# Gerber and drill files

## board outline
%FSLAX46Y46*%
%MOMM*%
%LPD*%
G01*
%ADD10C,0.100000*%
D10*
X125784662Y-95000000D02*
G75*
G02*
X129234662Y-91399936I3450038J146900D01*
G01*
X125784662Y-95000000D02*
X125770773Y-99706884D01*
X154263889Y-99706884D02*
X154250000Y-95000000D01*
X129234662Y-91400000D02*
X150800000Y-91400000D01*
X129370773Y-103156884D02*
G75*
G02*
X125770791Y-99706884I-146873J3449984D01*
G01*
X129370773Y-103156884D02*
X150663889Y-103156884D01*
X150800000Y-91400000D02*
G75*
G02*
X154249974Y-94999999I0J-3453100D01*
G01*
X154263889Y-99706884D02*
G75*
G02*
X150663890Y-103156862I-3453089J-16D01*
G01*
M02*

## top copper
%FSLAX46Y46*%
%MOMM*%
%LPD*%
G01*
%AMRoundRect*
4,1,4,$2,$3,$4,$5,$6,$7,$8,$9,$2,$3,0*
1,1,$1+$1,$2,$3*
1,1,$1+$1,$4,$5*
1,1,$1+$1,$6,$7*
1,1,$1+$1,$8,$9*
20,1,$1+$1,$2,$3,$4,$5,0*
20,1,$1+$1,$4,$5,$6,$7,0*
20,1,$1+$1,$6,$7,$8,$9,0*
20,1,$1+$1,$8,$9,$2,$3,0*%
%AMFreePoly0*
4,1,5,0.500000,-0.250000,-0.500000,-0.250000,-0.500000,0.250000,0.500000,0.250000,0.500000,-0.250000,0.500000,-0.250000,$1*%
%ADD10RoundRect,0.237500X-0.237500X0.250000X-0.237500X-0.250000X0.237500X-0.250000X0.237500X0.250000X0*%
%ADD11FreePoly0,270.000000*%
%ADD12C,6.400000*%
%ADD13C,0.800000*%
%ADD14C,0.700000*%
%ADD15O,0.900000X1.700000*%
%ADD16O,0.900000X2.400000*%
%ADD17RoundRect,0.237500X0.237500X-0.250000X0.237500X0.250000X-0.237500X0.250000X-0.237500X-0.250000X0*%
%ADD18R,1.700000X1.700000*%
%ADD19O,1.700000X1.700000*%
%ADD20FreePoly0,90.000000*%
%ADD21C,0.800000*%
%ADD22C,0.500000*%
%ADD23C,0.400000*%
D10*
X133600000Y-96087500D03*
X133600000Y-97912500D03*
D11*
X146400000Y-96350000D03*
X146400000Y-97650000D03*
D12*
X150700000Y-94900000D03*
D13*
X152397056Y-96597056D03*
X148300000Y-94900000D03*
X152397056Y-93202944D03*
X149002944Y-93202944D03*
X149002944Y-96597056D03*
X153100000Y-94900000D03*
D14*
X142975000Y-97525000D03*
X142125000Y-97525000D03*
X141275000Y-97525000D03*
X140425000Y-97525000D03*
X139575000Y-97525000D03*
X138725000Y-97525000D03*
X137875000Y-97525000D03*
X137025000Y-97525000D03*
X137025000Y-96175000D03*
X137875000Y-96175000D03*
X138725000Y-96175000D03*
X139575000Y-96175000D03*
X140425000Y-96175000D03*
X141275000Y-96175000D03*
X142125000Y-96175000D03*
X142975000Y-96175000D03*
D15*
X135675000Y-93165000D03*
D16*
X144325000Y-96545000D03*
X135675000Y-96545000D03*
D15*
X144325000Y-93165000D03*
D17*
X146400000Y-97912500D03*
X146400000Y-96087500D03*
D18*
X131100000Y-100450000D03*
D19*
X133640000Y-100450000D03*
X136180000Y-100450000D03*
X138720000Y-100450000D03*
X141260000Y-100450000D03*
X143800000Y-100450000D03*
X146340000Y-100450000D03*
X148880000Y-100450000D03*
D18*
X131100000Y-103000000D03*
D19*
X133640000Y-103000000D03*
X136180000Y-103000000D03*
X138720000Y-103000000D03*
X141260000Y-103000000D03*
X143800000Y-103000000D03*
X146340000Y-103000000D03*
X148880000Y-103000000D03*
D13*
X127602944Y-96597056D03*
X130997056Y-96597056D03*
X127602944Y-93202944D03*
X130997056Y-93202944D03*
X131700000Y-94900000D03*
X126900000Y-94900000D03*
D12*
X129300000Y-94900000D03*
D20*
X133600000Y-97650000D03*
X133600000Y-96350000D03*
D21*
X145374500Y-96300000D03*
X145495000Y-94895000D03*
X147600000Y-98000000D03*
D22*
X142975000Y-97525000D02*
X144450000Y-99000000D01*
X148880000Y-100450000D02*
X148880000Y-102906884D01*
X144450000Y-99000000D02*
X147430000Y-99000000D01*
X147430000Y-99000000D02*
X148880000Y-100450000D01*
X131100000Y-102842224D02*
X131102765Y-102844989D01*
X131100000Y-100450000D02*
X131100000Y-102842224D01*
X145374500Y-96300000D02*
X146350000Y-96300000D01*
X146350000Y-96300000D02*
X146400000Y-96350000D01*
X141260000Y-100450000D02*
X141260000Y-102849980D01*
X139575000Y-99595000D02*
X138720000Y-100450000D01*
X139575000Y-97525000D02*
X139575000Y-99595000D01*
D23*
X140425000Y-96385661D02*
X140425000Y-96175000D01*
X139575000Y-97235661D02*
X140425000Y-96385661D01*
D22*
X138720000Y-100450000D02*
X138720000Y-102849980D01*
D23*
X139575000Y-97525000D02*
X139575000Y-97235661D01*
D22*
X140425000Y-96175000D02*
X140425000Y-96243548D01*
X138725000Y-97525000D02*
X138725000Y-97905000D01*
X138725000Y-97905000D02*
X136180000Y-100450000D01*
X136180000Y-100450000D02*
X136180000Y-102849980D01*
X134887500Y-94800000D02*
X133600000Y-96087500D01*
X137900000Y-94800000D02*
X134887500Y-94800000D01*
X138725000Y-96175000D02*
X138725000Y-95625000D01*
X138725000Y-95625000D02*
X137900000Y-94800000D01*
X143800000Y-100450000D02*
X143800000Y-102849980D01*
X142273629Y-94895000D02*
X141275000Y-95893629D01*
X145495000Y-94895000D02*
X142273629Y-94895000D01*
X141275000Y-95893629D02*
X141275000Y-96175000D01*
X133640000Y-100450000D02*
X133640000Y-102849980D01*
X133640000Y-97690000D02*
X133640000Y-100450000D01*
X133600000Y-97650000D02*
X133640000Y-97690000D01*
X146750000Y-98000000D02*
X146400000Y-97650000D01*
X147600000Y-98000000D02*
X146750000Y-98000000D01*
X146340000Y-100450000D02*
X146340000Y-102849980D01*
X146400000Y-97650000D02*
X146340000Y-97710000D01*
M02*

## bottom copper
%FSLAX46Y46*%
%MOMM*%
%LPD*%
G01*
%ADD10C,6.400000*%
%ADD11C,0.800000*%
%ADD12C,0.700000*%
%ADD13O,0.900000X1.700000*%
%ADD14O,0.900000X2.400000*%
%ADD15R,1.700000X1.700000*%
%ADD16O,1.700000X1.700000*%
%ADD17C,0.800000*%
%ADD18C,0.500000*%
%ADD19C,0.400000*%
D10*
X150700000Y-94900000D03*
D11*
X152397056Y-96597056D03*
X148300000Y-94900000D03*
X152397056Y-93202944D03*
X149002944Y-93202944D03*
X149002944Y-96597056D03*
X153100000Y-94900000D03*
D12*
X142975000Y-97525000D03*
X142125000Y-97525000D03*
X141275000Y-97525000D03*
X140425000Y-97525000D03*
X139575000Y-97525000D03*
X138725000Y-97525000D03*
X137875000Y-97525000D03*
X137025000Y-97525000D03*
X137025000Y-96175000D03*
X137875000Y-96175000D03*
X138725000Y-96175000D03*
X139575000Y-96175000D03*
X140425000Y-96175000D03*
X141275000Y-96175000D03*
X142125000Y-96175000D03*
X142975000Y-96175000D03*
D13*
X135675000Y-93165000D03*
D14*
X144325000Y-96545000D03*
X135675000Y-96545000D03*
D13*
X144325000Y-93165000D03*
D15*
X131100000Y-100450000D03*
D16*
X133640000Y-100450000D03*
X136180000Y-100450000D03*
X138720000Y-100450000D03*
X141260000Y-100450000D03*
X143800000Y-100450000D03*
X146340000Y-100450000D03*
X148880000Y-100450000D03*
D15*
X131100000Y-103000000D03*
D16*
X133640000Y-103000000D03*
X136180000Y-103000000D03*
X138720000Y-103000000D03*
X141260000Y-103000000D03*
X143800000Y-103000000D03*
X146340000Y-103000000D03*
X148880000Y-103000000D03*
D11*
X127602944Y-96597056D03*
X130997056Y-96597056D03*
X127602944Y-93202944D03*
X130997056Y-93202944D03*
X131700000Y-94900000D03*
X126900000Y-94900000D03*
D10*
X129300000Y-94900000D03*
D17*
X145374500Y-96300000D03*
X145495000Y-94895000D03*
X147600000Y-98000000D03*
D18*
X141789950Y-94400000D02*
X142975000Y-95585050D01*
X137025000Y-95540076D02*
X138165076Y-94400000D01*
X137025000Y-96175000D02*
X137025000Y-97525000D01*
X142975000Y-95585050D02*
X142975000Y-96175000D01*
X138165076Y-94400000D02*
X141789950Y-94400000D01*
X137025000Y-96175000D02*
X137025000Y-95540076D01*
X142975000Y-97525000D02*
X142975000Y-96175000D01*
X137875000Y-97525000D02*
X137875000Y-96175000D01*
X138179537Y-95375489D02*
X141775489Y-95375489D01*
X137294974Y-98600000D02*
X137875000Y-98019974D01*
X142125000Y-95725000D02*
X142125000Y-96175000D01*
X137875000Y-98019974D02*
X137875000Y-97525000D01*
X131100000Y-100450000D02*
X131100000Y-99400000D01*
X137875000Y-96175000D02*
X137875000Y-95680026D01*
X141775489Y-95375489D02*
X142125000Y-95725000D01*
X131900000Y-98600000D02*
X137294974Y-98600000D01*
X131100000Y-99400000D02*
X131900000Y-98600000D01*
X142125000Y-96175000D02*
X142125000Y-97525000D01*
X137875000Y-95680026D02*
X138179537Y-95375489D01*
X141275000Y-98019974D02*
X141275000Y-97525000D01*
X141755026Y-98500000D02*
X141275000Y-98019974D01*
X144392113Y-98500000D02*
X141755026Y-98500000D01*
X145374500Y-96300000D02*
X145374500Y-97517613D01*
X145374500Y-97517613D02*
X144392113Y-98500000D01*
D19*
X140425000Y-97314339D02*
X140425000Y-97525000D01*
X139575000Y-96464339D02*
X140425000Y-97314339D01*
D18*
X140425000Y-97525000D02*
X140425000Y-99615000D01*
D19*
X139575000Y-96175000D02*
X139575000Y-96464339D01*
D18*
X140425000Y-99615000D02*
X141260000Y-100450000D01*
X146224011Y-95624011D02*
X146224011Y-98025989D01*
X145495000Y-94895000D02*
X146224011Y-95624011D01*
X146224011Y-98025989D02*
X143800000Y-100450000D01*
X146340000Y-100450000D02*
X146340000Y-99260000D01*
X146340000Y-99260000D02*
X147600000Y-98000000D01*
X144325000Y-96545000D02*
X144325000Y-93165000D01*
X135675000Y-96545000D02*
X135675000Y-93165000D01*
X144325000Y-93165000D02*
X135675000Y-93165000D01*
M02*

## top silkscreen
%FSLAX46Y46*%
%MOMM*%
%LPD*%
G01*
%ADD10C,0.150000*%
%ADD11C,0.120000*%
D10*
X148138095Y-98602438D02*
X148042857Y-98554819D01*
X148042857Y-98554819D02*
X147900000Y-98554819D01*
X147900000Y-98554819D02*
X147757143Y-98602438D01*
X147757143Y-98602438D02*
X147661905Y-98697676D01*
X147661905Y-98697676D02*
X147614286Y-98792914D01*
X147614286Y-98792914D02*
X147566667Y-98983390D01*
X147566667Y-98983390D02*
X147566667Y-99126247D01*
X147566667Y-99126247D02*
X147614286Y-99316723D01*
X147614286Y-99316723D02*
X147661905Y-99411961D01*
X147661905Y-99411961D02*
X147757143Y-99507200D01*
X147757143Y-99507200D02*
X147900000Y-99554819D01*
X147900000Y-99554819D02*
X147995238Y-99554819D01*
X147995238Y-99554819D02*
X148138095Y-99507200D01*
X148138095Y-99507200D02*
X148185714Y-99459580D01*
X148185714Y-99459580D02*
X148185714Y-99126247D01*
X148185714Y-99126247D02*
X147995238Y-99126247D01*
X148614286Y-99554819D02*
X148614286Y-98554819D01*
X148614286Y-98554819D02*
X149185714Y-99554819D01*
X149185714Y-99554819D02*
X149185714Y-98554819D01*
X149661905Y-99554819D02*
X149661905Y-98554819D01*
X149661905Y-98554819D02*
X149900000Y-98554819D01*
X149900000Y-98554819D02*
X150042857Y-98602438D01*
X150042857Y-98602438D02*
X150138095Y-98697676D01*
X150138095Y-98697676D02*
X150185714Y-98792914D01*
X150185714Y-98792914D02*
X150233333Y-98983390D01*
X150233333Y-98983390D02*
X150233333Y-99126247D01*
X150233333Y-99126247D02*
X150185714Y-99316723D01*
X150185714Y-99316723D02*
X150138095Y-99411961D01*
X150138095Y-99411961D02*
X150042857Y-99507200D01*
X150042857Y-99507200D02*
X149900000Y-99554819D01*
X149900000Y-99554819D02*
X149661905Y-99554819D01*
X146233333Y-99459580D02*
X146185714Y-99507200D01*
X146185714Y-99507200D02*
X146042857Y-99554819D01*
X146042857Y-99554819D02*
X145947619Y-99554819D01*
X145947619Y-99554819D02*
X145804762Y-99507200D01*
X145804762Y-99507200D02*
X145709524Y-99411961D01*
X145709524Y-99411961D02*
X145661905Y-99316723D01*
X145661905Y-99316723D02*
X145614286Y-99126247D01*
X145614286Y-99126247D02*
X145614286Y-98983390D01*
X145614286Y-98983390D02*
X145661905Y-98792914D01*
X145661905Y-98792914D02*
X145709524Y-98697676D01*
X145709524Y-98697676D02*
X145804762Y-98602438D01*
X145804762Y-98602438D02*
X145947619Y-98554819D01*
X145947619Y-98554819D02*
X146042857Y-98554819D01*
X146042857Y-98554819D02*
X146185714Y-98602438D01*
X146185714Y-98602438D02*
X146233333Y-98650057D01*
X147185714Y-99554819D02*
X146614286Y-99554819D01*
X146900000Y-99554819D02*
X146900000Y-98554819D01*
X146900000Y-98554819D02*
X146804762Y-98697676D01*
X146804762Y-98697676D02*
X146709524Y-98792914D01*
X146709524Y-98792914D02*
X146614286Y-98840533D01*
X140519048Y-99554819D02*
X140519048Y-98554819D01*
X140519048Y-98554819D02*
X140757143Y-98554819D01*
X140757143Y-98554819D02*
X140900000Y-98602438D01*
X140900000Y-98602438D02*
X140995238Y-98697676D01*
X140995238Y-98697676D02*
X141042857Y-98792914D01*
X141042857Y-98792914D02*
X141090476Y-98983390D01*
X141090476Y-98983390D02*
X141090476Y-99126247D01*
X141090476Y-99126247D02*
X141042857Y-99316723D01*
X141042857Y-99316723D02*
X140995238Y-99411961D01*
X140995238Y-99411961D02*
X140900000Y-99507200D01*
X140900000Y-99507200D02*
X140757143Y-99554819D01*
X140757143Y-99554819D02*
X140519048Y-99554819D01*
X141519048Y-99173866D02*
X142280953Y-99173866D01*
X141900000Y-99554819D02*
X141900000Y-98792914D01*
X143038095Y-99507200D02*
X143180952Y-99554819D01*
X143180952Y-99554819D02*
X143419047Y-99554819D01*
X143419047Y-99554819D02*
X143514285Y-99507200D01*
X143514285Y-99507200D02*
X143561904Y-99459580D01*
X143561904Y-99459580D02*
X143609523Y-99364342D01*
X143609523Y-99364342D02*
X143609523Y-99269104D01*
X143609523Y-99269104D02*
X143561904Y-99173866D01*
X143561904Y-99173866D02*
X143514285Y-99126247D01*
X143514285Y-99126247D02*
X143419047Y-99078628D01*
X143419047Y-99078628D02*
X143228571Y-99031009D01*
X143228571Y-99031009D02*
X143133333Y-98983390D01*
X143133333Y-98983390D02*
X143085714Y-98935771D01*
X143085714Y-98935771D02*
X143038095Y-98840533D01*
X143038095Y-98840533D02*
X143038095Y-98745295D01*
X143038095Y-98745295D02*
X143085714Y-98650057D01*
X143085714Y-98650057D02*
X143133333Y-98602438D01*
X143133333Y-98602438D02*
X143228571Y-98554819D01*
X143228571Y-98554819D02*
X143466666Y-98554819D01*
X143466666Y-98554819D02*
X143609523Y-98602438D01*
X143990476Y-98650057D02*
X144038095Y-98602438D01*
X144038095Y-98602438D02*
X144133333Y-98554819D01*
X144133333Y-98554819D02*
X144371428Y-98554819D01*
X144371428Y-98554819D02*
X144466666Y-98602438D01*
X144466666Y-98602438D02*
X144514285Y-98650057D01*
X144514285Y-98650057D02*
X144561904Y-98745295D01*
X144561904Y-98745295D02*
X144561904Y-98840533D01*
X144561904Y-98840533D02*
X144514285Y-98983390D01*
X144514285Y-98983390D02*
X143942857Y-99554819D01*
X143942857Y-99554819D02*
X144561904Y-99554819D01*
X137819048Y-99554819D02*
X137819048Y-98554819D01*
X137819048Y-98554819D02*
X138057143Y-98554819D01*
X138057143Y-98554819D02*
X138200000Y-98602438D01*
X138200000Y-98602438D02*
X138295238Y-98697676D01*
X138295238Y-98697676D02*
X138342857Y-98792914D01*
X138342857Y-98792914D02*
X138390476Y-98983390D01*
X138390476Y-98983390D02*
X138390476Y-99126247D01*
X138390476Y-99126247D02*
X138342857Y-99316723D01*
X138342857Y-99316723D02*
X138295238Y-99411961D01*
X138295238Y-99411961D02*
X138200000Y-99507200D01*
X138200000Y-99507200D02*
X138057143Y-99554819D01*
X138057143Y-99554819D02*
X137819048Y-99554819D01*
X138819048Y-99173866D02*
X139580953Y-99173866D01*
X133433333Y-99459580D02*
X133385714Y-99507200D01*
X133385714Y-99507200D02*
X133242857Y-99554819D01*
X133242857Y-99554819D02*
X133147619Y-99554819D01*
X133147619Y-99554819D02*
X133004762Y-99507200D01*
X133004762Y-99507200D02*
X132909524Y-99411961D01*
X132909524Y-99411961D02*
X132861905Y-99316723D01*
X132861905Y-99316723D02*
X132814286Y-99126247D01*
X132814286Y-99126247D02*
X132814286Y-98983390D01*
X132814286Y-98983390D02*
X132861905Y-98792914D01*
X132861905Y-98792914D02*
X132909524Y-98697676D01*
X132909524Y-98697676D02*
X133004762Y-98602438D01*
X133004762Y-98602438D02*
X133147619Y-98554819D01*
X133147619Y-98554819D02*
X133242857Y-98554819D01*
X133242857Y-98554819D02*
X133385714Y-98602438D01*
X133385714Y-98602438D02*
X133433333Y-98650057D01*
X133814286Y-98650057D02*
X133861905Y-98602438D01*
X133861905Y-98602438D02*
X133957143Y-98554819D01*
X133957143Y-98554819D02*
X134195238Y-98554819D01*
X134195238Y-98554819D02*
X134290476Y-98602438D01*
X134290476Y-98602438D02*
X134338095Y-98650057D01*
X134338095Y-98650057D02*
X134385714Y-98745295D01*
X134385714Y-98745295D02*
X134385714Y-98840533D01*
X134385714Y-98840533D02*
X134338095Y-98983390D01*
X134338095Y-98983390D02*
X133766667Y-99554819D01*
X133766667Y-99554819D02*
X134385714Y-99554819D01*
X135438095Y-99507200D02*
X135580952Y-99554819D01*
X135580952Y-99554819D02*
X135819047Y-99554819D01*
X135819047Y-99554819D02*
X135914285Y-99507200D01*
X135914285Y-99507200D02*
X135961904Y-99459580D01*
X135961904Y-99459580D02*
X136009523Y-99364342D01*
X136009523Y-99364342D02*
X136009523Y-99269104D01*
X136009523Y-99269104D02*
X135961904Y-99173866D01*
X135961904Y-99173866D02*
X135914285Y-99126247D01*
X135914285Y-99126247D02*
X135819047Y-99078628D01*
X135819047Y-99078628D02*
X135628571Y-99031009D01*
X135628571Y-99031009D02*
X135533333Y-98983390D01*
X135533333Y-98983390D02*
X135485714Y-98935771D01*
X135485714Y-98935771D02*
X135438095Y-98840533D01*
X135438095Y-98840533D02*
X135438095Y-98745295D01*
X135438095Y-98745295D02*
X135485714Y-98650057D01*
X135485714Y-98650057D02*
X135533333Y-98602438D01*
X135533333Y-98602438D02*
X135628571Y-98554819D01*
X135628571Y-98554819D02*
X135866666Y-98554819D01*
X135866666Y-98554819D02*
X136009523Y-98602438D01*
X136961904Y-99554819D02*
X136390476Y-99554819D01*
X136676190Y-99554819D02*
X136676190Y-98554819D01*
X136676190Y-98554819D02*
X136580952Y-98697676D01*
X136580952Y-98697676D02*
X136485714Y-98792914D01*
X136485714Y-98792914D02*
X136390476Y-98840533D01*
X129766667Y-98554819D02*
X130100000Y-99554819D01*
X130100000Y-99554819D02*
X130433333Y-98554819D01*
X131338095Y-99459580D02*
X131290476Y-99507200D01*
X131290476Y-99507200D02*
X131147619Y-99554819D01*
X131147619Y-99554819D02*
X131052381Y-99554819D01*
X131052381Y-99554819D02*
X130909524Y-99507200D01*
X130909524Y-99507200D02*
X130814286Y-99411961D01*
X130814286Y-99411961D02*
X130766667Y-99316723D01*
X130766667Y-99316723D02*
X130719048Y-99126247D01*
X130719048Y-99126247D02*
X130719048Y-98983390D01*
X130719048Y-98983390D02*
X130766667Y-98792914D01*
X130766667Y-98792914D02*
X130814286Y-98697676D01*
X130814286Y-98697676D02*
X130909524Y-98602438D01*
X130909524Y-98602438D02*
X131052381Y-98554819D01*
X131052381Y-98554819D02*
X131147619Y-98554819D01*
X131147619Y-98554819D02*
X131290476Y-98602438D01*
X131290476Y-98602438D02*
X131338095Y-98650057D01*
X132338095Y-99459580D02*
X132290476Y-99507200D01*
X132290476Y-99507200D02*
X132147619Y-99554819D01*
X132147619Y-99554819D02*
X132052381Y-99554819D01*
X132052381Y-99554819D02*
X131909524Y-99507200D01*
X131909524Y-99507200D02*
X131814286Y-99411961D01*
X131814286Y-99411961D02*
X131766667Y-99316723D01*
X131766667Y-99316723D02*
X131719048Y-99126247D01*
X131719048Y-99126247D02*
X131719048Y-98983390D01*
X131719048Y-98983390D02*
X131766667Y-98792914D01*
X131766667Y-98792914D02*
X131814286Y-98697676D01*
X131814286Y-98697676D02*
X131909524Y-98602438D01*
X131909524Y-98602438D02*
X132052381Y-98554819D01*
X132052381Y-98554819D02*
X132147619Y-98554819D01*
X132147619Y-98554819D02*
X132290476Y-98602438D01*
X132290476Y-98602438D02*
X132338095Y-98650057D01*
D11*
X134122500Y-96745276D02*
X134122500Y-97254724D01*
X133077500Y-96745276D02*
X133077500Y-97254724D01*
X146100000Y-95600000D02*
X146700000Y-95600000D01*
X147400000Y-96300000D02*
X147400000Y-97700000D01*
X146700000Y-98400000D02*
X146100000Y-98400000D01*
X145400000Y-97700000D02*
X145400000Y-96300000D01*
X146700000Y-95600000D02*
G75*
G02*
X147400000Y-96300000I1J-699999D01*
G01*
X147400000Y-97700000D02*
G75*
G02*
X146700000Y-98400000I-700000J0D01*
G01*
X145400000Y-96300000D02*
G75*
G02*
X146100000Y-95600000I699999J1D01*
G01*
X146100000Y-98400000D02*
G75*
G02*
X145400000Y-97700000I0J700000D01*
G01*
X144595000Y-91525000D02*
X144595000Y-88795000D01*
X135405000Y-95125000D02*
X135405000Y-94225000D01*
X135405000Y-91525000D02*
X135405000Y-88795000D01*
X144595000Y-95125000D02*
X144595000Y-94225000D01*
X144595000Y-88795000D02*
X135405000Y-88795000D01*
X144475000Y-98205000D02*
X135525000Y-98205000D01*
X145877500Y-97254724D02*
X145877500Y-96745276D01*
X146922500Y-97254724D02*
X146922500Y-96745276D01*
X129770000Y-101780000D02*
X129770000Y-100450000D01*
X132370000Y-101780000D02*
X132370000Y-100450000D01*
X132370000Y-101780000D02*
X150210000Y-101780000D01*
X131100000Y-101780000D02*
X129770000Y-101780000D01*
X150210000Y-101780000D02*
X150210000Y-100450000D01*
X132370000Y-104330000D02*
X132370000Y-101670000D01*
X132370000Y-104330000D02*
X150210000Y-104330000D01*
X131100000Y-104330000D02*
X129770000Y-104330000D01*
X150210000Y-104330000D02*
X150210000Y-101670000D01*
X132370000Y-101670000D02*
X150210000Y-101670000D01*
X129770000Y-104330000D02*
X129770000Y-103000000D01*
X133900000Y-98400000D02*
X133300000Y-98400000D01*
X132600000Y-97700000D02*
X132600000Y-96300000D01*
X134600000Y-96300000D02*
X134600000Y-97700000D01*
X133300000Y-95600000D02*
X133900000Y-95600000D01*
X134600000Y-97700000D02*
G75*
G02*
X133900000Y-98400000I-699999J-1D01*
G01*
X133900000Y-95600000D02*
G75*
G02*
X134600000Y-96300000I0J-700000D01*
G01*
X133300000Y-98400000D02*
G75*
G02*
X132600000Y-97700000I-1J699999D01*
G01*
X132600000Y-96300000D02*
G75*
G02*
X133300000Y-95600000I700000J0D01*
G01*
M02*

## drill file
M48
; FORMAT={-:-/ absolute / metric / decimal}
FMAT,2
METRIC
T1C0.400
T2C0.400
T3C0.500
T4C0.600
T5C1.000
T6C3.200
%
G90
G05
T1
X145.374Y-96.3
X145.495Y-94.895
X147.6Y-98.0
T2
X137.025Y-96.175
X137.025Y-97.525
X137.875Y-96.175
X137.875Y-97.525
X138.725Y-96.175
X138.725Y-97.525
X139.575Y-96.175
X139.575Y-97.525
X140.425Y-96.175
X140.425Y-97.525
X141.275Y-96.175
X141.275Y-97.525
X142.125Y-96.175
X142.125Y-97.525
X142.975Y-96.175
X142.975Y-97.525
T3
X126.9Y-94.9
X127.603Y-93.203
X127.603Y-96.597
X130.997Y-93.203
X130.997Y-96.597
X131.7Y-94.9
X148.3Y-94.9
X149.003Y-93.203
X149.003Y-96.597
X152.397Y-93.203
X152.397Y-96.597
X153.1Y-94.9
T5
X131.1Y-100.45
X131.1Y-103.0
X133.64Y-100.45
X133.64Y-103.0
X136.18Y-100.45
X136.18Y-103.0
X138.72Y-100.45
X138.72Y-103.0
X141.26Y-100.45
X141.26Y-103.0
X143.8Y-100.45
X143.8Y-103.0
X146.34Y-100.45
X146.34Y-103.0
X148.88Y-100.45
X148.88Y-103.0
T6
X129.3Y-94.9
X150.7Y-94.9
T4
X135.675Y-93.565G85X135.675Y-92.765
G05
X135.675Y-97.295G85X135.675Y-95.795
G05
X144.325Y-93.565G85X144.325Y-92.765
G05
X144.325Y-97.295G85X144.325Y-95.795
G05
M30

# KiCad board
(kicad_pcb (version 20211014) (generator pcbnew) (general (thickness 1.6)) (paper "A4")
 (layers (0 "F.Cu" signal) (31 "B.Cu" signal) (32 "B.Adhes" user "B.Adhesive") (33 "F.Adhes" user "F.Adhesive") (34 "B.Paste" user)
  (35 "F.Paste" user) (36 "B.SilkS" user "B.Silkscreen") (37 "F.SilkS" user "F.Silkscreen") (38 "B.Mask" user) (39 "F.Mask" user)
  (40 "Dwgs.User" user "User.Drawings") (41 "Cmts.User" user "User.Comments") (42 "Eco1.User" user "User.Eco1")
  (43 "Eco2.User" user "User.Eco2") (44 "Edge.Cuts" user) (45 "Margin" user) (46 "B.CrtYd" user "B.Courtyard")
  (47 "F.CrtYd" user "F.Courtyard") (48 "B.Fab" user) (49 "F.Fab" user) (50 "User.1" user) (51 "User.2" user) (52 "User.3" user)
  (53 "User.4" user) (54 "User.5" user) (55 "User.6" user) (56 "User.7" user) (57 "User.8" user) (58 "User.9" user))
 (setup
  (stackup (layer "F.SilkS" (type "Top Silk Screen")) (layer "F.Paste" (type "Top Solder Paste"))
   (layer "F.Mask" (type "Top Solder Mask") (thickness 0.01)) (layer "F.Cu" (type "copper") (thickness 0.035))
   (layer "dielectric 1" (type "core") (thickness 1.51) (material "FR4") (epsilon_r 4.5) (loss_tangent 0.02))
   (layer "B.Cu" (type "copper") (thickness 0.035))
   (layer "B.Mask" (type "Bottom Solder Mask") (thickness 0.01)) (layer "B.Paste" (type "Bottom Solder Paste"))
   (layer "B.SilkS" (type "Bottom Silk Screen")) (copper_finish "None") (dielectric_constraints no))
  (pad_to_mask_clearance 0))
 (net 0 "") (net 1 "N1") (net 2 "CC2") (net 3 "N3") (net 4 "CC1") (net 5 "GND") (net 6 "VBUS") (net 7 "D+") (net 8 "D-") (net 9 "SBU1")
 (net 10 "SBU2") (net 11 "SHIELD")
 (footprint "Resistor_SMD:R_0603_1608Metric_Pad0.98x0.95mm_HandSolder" (layer "F.Cu") (at 133.6 97 -90)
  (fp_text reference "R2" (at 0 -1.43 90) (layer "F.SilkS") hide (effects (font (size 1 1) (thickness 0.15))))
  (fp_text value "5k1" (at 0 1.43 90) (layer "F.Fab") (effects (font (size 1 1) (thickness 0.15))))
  (fp_line (start -0.254724 -0.5225) (end 0.254724 -0.5225) (layer "F.SilkS") (width 0.12))
  (fp_line (start -0.254724 0.5225) (end 0.254724 0.5225) (layer "F.SilkS") (width 0.12))
  (pad "1" smd roundrect (at -0.9125 0 270) (size 0.975 0.95) (layers "F.Cu" "F.Paste" "F.Mask") (roundrect_rratio 0.25) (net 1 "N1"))
  (pad "2" smd roundrect (at 0.9125 0 270) (size 0.975 0.95) (layers "F.Cu" "F.Paste" "F.Mask") (roundrect_rratio 0.25) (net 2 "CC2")))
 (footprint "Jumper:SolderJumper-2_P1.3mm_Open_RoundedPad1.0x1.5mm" (layer "F.Cu") (at 146.4 97 -90)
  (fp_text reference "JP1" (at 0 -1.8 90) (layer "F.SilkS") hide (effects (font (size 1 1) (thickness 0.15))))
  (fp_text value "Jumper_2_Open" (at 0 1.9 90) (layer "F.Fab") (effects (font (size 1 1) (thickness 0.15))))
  (fp_line (start -1.4 0.3) (end -1.4 -0.3) (layer "F.SilkS") (width 0.12))
  (fp_line (start -0.7 -1) (end 0.7 -1) (layer "F.SilkS") (width 0.12))
  (fp_line (start 1.4 -0.3) (end 1.4 0.3) (layer "F.SilkS") (width 0.12))
  (fp_line (start 0.7 1) (end -0.7 1) (layer "F.SilkS") (width 0.12))
  (fp_arc (start -1.4 -0.3) (mid -1.194975 -0.794975) (end -0.7 -1) (layer "F.SilkS") (width 0.12))
  (fp_arc (start 0.7 -1) (mid 1.194975 -0.794975) (end 1.4 -0.3) (layer "F.SilkS") (width 0.12))
  (fp_arc (start -0.7 1) (mid -1.194975 0.794975) (end -1.4 0.3) (layer "F.SilkS") (width 0.12))
  (fp_arc (start 1.4 0.3) (mid 1.194975 0.794975) (end 0.7 1) (layer "F.SilkS") (width 0.12))
  (pad "1" smd custom (at -0.65 0 270) (size 1 0.5) (layers "F.Cu" "F.Mask") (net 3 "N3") (zone_connect 2)
   (options (clearance outline) (anchor rect)) (primitives))
  (pad "2" smd custom (at 0.65 0 270) (size 1 0.5) (layers "F.Cu" "F.Mask") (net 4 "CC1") (zone_connect 2)
   (options (clearance outline) (anchor rect)) (primitives)))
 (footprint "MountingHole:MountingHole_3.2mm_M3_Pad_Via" (layer "F.Cu") (at 150.7 94.9)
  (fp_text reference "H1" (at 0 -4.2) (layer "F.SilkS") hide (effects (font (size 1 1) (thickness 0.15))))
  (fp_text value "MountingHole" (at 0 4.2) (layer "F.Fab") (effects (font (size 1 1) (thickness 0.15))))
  (pad "1" thru_hole circle (at 0 0) (size 6.4 6.4) (drill 3.2) (layers *.Cu *.Mask))
  (pad "1" thru_hole circle (at 1.697056 1.697056) (size 0.8 0.8) (drill 0.5) (layers *.Cu *.Mask))
  (pad "1" thru_hole circle (at -2.4 0) (size 0.8 0.8) (drill 0.5) (layers *.Cu *.Mask))
  (pad "1" thru_hole circle (at 1.697056 -1.697056) (size 0.8 0.8) (drill 0.5) (layers *.Cu *.Mask))
  (pad "1" thru_hole circle (at -1.697056 -1.697056) (size 0.8 0.8) (drill 0.5) (layers *.Cu *.Mask))
  (pad "1" thru_hole circle (at -1.697056 1.697056) (size 0.8 0.8) (drill 0.5) (layers *.Cu *.Mask))
  (pad "1" thru_hole circle (at 2.4 0) (size 0.8 0.8) (drill 0.5) (layers *.Cu *.Mask)))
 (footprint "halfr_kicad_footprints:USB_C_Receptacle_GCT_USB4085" (layer "F.Cu") (at 142.975 97.525 180)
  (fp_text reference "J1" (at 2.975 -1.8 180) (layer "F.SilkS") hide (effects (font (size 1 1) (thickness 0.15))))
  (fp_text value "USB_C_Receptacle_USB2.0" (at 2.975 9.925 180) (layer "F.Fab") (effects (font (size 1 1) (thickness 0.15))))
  (fp_line (start -1.62 6) (end -1.62 8.73) (layer "F.SilkS") (width 0.12))
  (fp_line (start 7.57 2.4) (end 7.57 3.3) (layer "F.SilkS") (width 0.12))
  (fp_line (start 7.57 6) (end 7.57 8.73) (layer "F.SilkS") (width 0.12))
  (fp_line (start -1.62 2.4) (end -1.62 3.3) (layer "F.SilkS") (width 0.12))
  (fp_line (start -1.62 8.73) (end 7.57 8.73) (layer "F.SilkS") (width 0.12))
  (fp_line (start -1.5 -0.68) (end 7.45 -0.68) (layer "F.SilkS") (width 0.12))
  (pad "A1" thru_hole circle (at 0 0 180) (size 0.7 0.7) (drill 0.4) (layers *.Cu *.Mask) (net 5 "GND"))
  (pad "A4" thru_hole circle (at 0.85 0 180) (size 0.7 0.7) (drill 0.4) (layers *.Cu *.Mask) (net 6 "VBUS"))
  (pad "A5" thru_hole circle (at 1.7 0 180) (size 0.7 0.7) (drill 0.4) (layers *.Cu *.Mask) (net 3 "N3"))
  (pad "A6" thru_hole circle (at 2.55 0 180) (size 0.7 0.7) (drill 0.4) (layers *.Cu *.Mask) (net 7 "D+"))
  (pad "A7" thru_hole circle (at 3.4 0 180) (size 0.7 0.7) (drill 0.4) (layers *.Cu *.Mask) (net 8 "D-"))
  (pad "A8" thru_hole circle (at 4.25 0 180) (size 0.7 0.7) (drill 0.4) (layers *.Cu *.Mask) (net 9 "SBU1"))
  (pad "A9" thru_hole circle (at 5.1 0 180) (size 0.7 0.7) (drill 0.4) (layers *.Cu *.Mask) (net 6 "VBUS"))
  (pad "A12" thru_hole circle (at 5.95 0 180) (size 0.7 0.7) (drill 0.4) (layers *.Cu *.Mask) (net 5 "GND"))
  (pad "B1" thru_hole circle (at 5.95 1.35 180) (size 0.7 0.7) (drill 0.4) (layers *.Cu *.Mask) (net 5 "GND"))
  (pad "B4" thru_hole circle (at 5.1 1.35 180) (size 0.7 0.7) (drill 0.4) (layers *.Cu *.Mask) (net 6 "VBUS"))
  (pad "B5" thru_hole circle (at 4.25 1.35 180) (size 0.7 0.7) (drill 0.4) (layers *.Cu *.Mask) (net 1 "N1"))
  (pad "B6" thru_hole circle (at 3.4 1.35 180) (size 0.7 0.7) (drill 0.4) (layers *.Cu *.Mask) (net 7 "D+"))
  (pad "B7" thru_hole circle (at 2.55 1.35 180) (size 0.7 0.7) (drill 0.4) (layers *.Cu *.Mask) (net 8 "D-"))
  (pad "B8" thru_hole circle (at 1.7 1.35 180) (size 0.7 0.7) (drill 0.4) (layers *.Cu *.Mask) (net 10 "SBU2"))
  (pad "B9" thru_hole circle (at 0.85 1.35 180) (size 0.7 0.7) (drill 0.4) (layers *.Cu *.Mask) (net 6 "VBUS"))
  (pad "B12" thru_hole circle (at 0 1.35 180) (size 0.7 0.7) (drill 0.4) (layers *.Cu *.Mask) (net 5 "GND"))
  (pad "S1" thru_hole oval (at 7.3 4.36 180) (size 0.9 1.7) (drill oval 0.6 1.4) (layers *.Cu *.Mask) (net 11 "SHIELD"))
  (pad "S1" thru_hole oval (at -1.35 0.98 180) (size 0.9 2.4) (drill oval 0.6 2.1) (layers *.Cu *.Mask) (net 11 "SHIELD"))
  (pad "S1" thru_hole oval (at 7.3 0.98 180) (size 0.9 2.4) (drill oval 0.6 2.1) (layers *.Cu *.Mask) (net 11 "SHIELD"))
  (pad "S1" thru_hole oval (at -1.35 4.36 180) (size 0.9 1.7) (drill oval 0.6 1.4) (layers *.Cu *.Mask) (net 11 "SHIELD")))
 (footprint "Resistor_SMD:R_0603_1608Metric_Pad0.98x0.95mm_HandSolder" (layer "F.Cu") (at 146.4 97 90)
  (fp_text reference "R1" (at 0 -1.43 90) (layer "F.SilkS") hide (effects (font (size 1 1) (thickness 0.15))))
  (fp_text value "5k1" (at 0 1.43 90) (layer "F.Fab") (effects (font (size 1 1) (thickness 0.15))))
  (fp_line (start -0.254724 -0.5225) (end 0.254724 -0.5225) (layer "F.SilkS") (width 0.12))
  (fp_line (start -0.254724 0.5225) (end 0.254724 0.5225) (layer "F.SilkS") (width 0.12))
  (pad "1" smd roundrect (at -0.9125 0 90) (size 0.975 0.95) (layers "F.Cu" "F.Paste" "F.Mask") (roundrect_rratio 0.25) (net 4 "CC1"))
  (pad "2" smd roundrect (at 0.9125 0 90) (size 0.975 0.95) (layers "F.Cu" "F.Paste" "F.Mask") (roundrect_rratio 0.25) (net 3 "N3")))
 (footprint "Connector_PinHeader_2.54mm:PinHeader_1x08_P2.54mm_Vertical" (layer "F.Cu") (at 131.1 100.45 90)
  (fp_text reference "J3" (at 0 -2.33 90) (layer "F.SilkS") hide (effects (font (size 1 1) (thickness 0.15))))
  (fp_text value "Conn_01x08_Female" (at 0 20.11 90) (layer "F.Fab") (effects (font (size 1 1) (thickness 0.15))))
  (fp_line (start -1.33 -1.33) (end 0 -1.33) (layer "F.SilkS") (width 0.12))
  (fp_line (start -1.33 1.27) (end 0 1.27) (layer "F.SilkS") (width 0.12))
  (fp_line (start -1.33 1.27) (end -1.33 19.11) (layer "F.SilkS") (width 0.12))
  (fp_line (start -1.33 0) (end -1.33 -1.33) (layer "F.SilkS") (width 0.12))
  (fp_line (start -1.33 19.11) (end 0 19.11) (layer "F.SilkS") (width 0.12))
  (pad "1" thru_hole rect (at 0 0 90) (size 1.7 1.7) (drill 1) (layers *.Cu *.Mask) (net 6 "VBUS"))
  (pad "2" thru_hole oval (at 0 2.54 90) (size 1.7 1.7) (drill 1) (layers *.Cu *.Mask) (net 2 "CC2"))
  (pad "3" thru_hole oval (at 0 5.08 90) (size 1.7 1.7) (drill 1) (layers *.Cu *.Mask) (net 9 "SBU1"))
  (pad "4" thru_hole oval (at 0 7.62 90) (size 1.7 1.7) (drill 1) (layers *.Cu *.Mask) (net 8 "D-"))
  (pad "5" thru_hole oval (at 0 10.16 90) (size 1.7 1.7) (drill 1) (layers *.Cu *.Mask) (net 7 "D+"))
  (pad "6" thru_hole oval (at 0 12.7 90) (size 1.7 1.7) (drill 1) (layers *.Cu *.Mask) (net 10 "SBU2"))
  (pad "7" thru_hole oval (at 0 15.24 90) (size 1.7 1.7) (drill 1) (layers *.Cu *.Mask) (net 4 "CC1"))
  (pad "8" thru_hole oval (at 0 17.78 90) (size 1.7 1.7) (drill 1) (layers *.Cu *.Mask) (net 5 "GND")))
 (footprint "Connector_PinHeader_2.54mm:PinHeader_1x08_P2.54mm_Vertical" (layer "F.Cu") (at 131.1 103 90)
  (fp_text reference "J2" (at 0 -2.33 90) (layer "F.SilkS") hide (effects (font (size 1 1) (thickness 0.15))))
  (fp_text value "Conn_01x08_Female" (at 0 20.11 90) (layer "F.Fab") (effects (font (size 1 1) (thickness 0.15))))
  (fp_line (start -1.33 1.27) (end 1.33 1.27) (layer "F.SilkS") (width 0.12))
  (fp_line (start -1.33 1.27) (end -1.33 19.11) (layer "F.SilkS") (width 0.12))
  (fp_line (start -1.33 0) (end -1.33 -1.33) (layer "F.SilkS") (width 0.12))
  (fp_line (start -1.33 19.11) (end 1.33 19.11) (layer "F.SilkS") (width 0.12))
  (fp_line (start 1.33 1.27) (end 1.33 19.11) (layer "F.SilkS") (width 0.12))
  (fp_line (start -1.33 -1.33) (end 0 -1.33) (layer "F.SilkS") (width 0.12))
  (pad "1" thru_hole rect (at 0 0 90) (size 1.7 1.7) (drill 1) (layers *.Cu *.Mask) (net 6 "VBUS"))
  (pad "2" thru_hole oval (at 0 2.54 90) (size 1.7 1.7) (drill 1) (layers *.Cu *.Mask) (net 2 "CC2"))
  (pad "3" thru_hole oval (at 0 5.08 90) (size 1.7 1.7) (drill 1) (layers *.Cu *.Mask) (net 9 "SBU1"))
  (pad "4" thru_hole oval (at 0 7.62 90) (size 1.7 1.7) (drill 1) (layers *.Cu *.Mask) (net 8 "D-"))
  (pad "5" thru_hole oval (at 0 10.16 90) (size 1.7 1.7) (drill 1) (layers *.Cu *.Mask) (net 7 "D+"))
  (pad "6" thru_hole oval (at 0 12.7 90) (size 1.7 1.7) (drill 1) (layers *.Cu *.Mask) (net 10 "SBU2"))
  (pad "7" thru_hole oval (at 0 15.24 90) (size 1.7 1.7) (drill 1) (layers *.Cu *.Mask) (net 4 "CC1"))
  (pad "8" thru_hole oval (at 0 17.78 90) (size 1.7 1.7) (drill 1) (layers *.Cu *.Mask) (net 5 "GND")))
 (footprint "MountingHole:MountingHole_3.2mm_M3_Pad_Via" (layer "F.Cu") (at 129.3 94.9)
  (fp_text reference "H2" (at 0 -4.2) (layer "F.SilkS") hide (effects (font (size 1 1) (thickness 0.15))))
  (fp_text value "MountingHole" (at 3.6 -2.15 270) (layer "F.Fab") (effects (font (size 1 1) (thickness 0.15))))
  (pad "1" thru_hole circle (at -1.697056 1.697056) (size 0.8 0.8) (drill 0.5) (layers *.Cu *.Mask))
  (pad "1" thru_hole circle (at 1.697056 1.697056) (size 0.8 0.8) (drill 0.5) (layers *.Cu *.Mask))
  (pad "1" thru_hole circle (at -1.697056 -1.697056) (size 0.8 0.8) (drill 0.5) (layers *.Cu *.Mask))
  (pad "1" thru_hole circle (at 1.697056 -1.697056) (size 0.8 0.8) (drill 0.5) (layers *.Cu *.Mask))
  (pad "1" thru_hole circle (at 2.4 0) (size 0.8 0.8) (drill 0.5) (layers *.Cu *.Mask))
  (pad "1" thru_hole circle (at -2.4 0) (size 0.8 0.8) (drill 0.5) (layers *.Cu *.Mask))
  (pad "1" thru_hole circle (at 0 0) (size 6.4 6.4) (drill 3.2) (layers *.Cu *.Mask)))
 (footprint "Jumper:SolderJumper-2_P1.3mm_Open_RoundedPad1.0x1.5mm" (layer "F.Cu") (at 133.6 97 90)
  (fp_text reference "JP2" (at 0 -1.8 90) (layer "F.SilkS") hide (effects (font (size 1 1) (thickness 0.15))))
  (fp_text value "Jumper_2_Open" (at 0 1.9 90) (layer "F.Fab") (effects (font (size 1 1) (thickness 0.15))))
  (fp_line (start -1.4 0.3) (end -1.4 -0.3) (layer "F.SilkS") (width 0.12))
  (fp_line (start -0.7 -1) (end 0.7 -1) (layer "F.SilkS") (width 0.12))
  (fp_line (start 0.7 1) (end -0.7 1) (layer "F.SilkS") (width 0.12))
  (fp_line (start 1.4 -0.3) (end 1.4 0.3) (layer "F.SilkS") (width 0.12))
  (fp_arc (start -0.7 1) (mid -1.194975 0.794975) (end -1.4 0.3) (layer "F.SilkS") (width 0.12))
  (fp_arc (start 1.4 0.3) (mid 1.194975 0.794975) (end 0.7 1) (layer "F.SilkS") (width 0.12))
  (fp_arc (start -1.4 -0.3) (mid -1.194975 -0.794975) (end -0.7 -1) (layer "F.SilkS") (width 0.12))
  (fp_arc (start 0.7 -1) (mid 1.194975 -0.794975) (end 1.4 -0.3) (layer "F.SilkS") (width 0.12))
  (pad "1" smd custom (at -0.65 0 90) (size 1 0.5) (layers "F.Cu" "F.Mask") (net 2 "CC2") (zone_connect 2)
   (options (clearance outline) (anchor rect)) (primitives))
  (pad "2" smd custom (at 0.65 0 90) (size 1 0.5) (layers "F.Cu" "F.Mask") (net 1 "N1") (zone_connect 2)
   (options (clearance outline) (anchor rect)) (primitives)))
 (gr_arc (start 125.784662 95) (mid 126.741546 92.463889) (end 129.234662 91.4) (layer "Edge.Cuts") (width 0.1))
 (gr_line (start 125.784662 95) (end 125.770773 99.706884) (layer "Edge.Cuts") (width 0.1))
 (gr_line (start 154.263889 99.706884) (end 154.25 95) (layer "Edge.Cuts") (width 0.1))
 (gr_line (start 129.234662 91.4) (end 150.8 91.4) (layer "Edge.Cuts") (width 0.1))
 (gr_arc (start 129.370773 103.156884) (mid 126.834662 102.2) (end 125.770773 99.706884) (layer "Edge.Cuts") (width 0.1))
 (gr_line (start 129.370773 103.156884) (end 150.663889 103.156884) (layer "Edge.Cuts") (width 0.1))
 (gr_arc (start 150.8 91.4) (mid 153.293116 92.463889) (end 154.25 95) (layer "Edge.Cuts") (width 0.1))
 (gr_arc (start 154.263889 99.706884) (mid 153.2 102.2) (end 150.663889 103.156884) (layer "Edge.Cuts") (width 0.1))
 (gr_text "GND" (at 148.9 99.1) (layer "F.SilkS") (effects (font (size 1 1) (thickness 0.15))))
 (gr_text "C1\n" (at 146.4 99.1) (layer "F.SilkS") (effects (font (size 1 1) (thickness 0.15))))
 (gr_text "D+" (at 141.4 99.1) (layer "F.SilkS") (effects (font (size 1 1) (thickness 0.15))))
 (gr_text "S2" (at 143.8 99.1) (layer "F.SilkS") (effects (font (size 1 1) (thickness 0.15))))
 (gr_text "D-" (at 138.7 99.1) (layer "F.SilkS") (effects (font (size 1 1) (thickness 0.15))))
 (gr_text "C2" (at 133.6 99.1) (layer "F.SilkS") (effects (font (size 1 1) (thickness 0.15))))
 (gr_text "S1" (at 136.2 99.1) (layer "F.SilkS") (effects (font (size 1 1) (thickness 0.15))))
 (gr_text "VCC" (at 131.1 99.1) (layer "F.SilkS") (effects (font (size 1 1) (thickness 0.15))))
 (segment (start 142.975 97.525) (end 144.45 99) (width 0.5) (layer "F.Cu") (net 5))
 (segment (start 148.88 100.45) (end 148.88 102.906884) (width 0.5) (layer "F.Cu") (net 5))
 (segment (start 144.45 99) (end 147.43 99) (width 0.5) (layer "F.Cu") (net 5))
 (segment (start 147.43 99) (end 148.88 100.45) (width 0.5) (layer "F.Cu") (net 5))
 (segment (start 141.78995 94.4) (end 142.975 95.58505) (width 0.5) (layer "B.Cu") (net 5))
 (segment (start 137.025 95.540076) (end 138.165076 94.4) (width 0.5) (layer "B.Cu") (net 5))
 (segment (start 137.025 96.175) (end 137.025 97.525) (width 0.5) (layer "B.Cu") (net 5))
 (segment (start 142.975 95.58505) (end 142.975 96.175) (width 0.5) (layer "B.Cu") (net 5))
 (segment (start 138.165076 94.4) (end 141.78995 94.4) (width 0.5) (layer "B.Cu") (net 5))
 (segment (start 137.025 96.175) (end 137.025 95.540076) (width 0.5) (layer "B.Cu") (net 5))
 (segment (start 142.975 97.525) (end 142.975 96.175) (width 0.5) (layer "B.Cu") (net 5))
 (segment (start 131.1 102.842224) (end 131.102765 102.844989) (width 0.5) (layer "F.Cu") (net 6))
 (segment (start 131.1 100.45) (end 131.1 102.842224) (width 0.5) (layer "F.Cu") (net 6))
 (segment (start 137.875 97.525) (end 137.875 96.175) (width 0.5) (layer "B.Cu") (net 6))
 (segment (start 138.179537 95.375489) (end 141.775489 95.375489) (width 0.5) (layer "B.Cu") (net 6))
 (segment (start 137.294974 98.6) (end 137.875 98.019974) (width 0.5) (layer "B.Cu") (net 6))
 (segment (start 142.125 95.725) (end 142.125 96.175) (width 0.5) (layer "B.Cu") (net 6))
 (segment (start 137.875 98.019974) (end 137.875 97.525) (width 0.5) (layer "B.Cu") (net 6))
 (segment (start 131.1 100.45) (end 131.1 99.4) (width 0.5) (layer "B.Cu") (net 6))
 (segment (start 137.875 96.175) (end 137.875 95.680026) (width 0.5) (layer "B.Cu") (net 6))
 (segment (start 141.775489 95.375489) (end 142.125 95.725) (width 0.5) (layer "B.Cu") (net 6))
 (segment (start 131.9 98.6) (end 137.294974 98.6) (width 0.5) (layer "B.Cu") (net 6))
 (segment (start 131.1 99.4) (end 131.9 98.6) (width 0.5) (layer "B.Cu") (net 6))
 (segment (start 142.125 96.175) (end 142.125 97.525) (width 0.5) (layer "B.Cu") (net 6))
 (segment (start 137.875 95.680026) (end 138.179537 95.375489) (width 0.5) (layer "B.Cu") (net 6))
 (segment (start 145.3745 96.3) (end 146.35 96.3) (width 0.5) (layer "F.Cu") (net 3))
 (segment (start 146.35 96.3) (end 146.4 96.35) (width 0.5) (layer "F.Cu") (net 3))
 (via (at 145.3745 96.3) (size 0.8) (drill 0.4) (layers "F.Cu" "B.Cu") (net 3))
 (segment (start 141.275 98.019974) (end 141.275 97.525) (width 0.5) (layer "B.Cu") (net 3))
 (segment (start 141.755026 98.5) (end 141.275 98.019974) (width 0.5) (layer "B.Cu") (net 3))
 (segment (start 144.392113 98.5) (end 141.755026 98.5) (width 0.5) (layer "B.Cu") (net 3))
 (segment (start 145.3745 96.3) (end 145.3745 97.517613) (width 0.5) (layer "B.Cu") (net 3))
 (segment (start 145.3745 97.517613) (end 144.392113 98.5) (width 0.5) (layer "B.Cu") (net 3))
 (segment (start 141.26 100.45) (end 141.26 102.84998) (width 0.5) (layer "F.Cu") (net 7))
 (segment (start 140.425 97.314339) (end 140.425 97.525) (width 0.4) (layer "B.Cu") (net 7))
 (segment (start 139.575 96.464339) (end 140.425 97.314339) (width 0.4) (layer "B.Cu") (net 7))
 (segment (start 140.425 97.525) (end 140.425 99.615) (width 0.5) (layer "B.Cu") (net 7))
 (segment (start 139.575 96.175) (end 139.575 96.464339) (width 0.4) (layer "B.Cu") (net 7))
 (segment (start 140.425 99.615) (end 141.26 100.45) (width 0.5) (layer "B.Cu") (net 7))
 (segment (start 139.575 99.595) (end 138.72 100.45) (width 0.5) (layer "F.Cu") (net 8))
 (segment (start 139.575 97.525) (end 139.575 99.595) (width 0.5) (layer "F.Cu") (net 8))
 (segment (start 140.425 96.385661) (end 140.425 96.175) (width 0.4) (layer "F.Cu") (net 8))
 (segment (start 139.575 97.235661) (end 140.425 96.385661) (width 0.4) (layer "F.Cu") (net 8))
 (segment (start 138.72 100.45) (end 138.72 102.84998) (width 0.5) (layer "F.Cu") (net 8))
 (segment (start 139.575 97.525) (end 139.575 97.235661) (width 0.4) (layer "F.Cu") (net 8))
 (segment (start 140.425 96.175) (end 140.425 96.243548) (width 0.5) (layer "F.Cu") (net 8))
 (segment (start 138.725 97.525) (end 138.725 97.905) (width 0.5) (layer "F.Cu") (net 9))
 (segment (start 138.725 97.905) (end 136.18 100.45) (width 0.5) (layer "F.Cu") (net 9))
 (segment (start 136.18 100.45) (end 136.18 102.84998) (width 0.5) (layer "F.Cu") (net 9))
 (segment (start 134.8875 94.8) (end 133.6 96.0875) (width 0.5) (layer "F.Cu") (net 1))
 (segment (start 137.9 94.8) (end 134.8875 94.8) (width 0.5) (layer "F.Cu") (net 1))
 (segment (start 138.725 96.175) (end 138.725 95.625) (width 0.5) (layer "F.Cu") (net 1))
 (segment (start 138.725 95.625) (end 137.9 94.8) (width 0.5) (layer "F.Cu") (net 1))
 (segment (start 143.8 100.45) (end 143.8 102.84998) (width 0.5) (layer "F.Cu") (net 10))
 (segment (start 142.273629 94.895) (end 141.275 95.893629) (width 0.5) (layer "F.Cu") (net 10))
 (segment (start 145.495 94.895) (end 142.273629 94.895) (width 0.5) (layer "F.Cu") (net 10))
 (segment (start 141.275 95.893629) (end 141.275 96.175) (width 0.5) (layer "F.Cu") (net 10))
 (via (at 145.495 94.895) (size 0.8) (drill 0.4) (layers "F.Cu" "B.Cu") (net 10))
 (segment (start 146.224011 95.624011) (end 146.224011 98.025989) (width 0.5) (layer "B.Cu") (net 10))
 (segment (start 145.495 94.895) (end 146.224011 95.624011) (width 0.5) (layer "B.Cu") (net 10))
 (segment (start 146.224011 98.025989) (end 143.8 100.45) (width 0.5) (layer "B.Cu") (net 10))
 (segment (start 133.64 100.45) (end 133.64 102.84998) (width 0.5) (layer "F.Cu") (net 2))
 (segment (start 133.64 97.69) (end 133.64 100.45) (width 0.5) (layer "F.Cu") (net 2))
 (segment (start 133.6 97.65) (end 133.64 97.69) (width 0.5) (layer "F.Cu") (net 2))
 (segment (start 146.75 98) (end 146.4 97.65) (width 0.5) (layer "F.Cu") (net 4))
 (segment (start 147.6 98) (end 146.75 98) (width 0.5) (layer "F.Cu") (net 4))
 (segment (start 146.34 100.45) (end 146.34 102.84998) (width 0.5) (layer "F.Cu") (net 4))
 (segment (start 146.4 97.65) (end 146.34 97.71) (width 0.5) (layer "F.Cu") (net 4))
 (via (at 147.6 98) (size 0.8) (drill 0.4) (layers "F.Cu" "B.Cu") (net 4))
 (segment (start 146.34 100.45) (end 146.34 99.26) (width 0.5) (layer "B.Cu") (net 4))
 (segment (start 146.34 99.26) (end 147.6 98) (width 0.5) (layer "B.Cu") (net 4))
 (segment (start 144.325 96.545) (end 144.325 93.165) (width 0.5) (layer "B.Cu") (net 11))
 (segment (start 135.675 96.545) (end 135.675 93.165) (width 0.5) (layer "B.Cu") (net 11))
 (segment (start 144.325 93.165) (end 135.675 93.165) (width 0.5) (layer "B.Cu") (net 11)))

